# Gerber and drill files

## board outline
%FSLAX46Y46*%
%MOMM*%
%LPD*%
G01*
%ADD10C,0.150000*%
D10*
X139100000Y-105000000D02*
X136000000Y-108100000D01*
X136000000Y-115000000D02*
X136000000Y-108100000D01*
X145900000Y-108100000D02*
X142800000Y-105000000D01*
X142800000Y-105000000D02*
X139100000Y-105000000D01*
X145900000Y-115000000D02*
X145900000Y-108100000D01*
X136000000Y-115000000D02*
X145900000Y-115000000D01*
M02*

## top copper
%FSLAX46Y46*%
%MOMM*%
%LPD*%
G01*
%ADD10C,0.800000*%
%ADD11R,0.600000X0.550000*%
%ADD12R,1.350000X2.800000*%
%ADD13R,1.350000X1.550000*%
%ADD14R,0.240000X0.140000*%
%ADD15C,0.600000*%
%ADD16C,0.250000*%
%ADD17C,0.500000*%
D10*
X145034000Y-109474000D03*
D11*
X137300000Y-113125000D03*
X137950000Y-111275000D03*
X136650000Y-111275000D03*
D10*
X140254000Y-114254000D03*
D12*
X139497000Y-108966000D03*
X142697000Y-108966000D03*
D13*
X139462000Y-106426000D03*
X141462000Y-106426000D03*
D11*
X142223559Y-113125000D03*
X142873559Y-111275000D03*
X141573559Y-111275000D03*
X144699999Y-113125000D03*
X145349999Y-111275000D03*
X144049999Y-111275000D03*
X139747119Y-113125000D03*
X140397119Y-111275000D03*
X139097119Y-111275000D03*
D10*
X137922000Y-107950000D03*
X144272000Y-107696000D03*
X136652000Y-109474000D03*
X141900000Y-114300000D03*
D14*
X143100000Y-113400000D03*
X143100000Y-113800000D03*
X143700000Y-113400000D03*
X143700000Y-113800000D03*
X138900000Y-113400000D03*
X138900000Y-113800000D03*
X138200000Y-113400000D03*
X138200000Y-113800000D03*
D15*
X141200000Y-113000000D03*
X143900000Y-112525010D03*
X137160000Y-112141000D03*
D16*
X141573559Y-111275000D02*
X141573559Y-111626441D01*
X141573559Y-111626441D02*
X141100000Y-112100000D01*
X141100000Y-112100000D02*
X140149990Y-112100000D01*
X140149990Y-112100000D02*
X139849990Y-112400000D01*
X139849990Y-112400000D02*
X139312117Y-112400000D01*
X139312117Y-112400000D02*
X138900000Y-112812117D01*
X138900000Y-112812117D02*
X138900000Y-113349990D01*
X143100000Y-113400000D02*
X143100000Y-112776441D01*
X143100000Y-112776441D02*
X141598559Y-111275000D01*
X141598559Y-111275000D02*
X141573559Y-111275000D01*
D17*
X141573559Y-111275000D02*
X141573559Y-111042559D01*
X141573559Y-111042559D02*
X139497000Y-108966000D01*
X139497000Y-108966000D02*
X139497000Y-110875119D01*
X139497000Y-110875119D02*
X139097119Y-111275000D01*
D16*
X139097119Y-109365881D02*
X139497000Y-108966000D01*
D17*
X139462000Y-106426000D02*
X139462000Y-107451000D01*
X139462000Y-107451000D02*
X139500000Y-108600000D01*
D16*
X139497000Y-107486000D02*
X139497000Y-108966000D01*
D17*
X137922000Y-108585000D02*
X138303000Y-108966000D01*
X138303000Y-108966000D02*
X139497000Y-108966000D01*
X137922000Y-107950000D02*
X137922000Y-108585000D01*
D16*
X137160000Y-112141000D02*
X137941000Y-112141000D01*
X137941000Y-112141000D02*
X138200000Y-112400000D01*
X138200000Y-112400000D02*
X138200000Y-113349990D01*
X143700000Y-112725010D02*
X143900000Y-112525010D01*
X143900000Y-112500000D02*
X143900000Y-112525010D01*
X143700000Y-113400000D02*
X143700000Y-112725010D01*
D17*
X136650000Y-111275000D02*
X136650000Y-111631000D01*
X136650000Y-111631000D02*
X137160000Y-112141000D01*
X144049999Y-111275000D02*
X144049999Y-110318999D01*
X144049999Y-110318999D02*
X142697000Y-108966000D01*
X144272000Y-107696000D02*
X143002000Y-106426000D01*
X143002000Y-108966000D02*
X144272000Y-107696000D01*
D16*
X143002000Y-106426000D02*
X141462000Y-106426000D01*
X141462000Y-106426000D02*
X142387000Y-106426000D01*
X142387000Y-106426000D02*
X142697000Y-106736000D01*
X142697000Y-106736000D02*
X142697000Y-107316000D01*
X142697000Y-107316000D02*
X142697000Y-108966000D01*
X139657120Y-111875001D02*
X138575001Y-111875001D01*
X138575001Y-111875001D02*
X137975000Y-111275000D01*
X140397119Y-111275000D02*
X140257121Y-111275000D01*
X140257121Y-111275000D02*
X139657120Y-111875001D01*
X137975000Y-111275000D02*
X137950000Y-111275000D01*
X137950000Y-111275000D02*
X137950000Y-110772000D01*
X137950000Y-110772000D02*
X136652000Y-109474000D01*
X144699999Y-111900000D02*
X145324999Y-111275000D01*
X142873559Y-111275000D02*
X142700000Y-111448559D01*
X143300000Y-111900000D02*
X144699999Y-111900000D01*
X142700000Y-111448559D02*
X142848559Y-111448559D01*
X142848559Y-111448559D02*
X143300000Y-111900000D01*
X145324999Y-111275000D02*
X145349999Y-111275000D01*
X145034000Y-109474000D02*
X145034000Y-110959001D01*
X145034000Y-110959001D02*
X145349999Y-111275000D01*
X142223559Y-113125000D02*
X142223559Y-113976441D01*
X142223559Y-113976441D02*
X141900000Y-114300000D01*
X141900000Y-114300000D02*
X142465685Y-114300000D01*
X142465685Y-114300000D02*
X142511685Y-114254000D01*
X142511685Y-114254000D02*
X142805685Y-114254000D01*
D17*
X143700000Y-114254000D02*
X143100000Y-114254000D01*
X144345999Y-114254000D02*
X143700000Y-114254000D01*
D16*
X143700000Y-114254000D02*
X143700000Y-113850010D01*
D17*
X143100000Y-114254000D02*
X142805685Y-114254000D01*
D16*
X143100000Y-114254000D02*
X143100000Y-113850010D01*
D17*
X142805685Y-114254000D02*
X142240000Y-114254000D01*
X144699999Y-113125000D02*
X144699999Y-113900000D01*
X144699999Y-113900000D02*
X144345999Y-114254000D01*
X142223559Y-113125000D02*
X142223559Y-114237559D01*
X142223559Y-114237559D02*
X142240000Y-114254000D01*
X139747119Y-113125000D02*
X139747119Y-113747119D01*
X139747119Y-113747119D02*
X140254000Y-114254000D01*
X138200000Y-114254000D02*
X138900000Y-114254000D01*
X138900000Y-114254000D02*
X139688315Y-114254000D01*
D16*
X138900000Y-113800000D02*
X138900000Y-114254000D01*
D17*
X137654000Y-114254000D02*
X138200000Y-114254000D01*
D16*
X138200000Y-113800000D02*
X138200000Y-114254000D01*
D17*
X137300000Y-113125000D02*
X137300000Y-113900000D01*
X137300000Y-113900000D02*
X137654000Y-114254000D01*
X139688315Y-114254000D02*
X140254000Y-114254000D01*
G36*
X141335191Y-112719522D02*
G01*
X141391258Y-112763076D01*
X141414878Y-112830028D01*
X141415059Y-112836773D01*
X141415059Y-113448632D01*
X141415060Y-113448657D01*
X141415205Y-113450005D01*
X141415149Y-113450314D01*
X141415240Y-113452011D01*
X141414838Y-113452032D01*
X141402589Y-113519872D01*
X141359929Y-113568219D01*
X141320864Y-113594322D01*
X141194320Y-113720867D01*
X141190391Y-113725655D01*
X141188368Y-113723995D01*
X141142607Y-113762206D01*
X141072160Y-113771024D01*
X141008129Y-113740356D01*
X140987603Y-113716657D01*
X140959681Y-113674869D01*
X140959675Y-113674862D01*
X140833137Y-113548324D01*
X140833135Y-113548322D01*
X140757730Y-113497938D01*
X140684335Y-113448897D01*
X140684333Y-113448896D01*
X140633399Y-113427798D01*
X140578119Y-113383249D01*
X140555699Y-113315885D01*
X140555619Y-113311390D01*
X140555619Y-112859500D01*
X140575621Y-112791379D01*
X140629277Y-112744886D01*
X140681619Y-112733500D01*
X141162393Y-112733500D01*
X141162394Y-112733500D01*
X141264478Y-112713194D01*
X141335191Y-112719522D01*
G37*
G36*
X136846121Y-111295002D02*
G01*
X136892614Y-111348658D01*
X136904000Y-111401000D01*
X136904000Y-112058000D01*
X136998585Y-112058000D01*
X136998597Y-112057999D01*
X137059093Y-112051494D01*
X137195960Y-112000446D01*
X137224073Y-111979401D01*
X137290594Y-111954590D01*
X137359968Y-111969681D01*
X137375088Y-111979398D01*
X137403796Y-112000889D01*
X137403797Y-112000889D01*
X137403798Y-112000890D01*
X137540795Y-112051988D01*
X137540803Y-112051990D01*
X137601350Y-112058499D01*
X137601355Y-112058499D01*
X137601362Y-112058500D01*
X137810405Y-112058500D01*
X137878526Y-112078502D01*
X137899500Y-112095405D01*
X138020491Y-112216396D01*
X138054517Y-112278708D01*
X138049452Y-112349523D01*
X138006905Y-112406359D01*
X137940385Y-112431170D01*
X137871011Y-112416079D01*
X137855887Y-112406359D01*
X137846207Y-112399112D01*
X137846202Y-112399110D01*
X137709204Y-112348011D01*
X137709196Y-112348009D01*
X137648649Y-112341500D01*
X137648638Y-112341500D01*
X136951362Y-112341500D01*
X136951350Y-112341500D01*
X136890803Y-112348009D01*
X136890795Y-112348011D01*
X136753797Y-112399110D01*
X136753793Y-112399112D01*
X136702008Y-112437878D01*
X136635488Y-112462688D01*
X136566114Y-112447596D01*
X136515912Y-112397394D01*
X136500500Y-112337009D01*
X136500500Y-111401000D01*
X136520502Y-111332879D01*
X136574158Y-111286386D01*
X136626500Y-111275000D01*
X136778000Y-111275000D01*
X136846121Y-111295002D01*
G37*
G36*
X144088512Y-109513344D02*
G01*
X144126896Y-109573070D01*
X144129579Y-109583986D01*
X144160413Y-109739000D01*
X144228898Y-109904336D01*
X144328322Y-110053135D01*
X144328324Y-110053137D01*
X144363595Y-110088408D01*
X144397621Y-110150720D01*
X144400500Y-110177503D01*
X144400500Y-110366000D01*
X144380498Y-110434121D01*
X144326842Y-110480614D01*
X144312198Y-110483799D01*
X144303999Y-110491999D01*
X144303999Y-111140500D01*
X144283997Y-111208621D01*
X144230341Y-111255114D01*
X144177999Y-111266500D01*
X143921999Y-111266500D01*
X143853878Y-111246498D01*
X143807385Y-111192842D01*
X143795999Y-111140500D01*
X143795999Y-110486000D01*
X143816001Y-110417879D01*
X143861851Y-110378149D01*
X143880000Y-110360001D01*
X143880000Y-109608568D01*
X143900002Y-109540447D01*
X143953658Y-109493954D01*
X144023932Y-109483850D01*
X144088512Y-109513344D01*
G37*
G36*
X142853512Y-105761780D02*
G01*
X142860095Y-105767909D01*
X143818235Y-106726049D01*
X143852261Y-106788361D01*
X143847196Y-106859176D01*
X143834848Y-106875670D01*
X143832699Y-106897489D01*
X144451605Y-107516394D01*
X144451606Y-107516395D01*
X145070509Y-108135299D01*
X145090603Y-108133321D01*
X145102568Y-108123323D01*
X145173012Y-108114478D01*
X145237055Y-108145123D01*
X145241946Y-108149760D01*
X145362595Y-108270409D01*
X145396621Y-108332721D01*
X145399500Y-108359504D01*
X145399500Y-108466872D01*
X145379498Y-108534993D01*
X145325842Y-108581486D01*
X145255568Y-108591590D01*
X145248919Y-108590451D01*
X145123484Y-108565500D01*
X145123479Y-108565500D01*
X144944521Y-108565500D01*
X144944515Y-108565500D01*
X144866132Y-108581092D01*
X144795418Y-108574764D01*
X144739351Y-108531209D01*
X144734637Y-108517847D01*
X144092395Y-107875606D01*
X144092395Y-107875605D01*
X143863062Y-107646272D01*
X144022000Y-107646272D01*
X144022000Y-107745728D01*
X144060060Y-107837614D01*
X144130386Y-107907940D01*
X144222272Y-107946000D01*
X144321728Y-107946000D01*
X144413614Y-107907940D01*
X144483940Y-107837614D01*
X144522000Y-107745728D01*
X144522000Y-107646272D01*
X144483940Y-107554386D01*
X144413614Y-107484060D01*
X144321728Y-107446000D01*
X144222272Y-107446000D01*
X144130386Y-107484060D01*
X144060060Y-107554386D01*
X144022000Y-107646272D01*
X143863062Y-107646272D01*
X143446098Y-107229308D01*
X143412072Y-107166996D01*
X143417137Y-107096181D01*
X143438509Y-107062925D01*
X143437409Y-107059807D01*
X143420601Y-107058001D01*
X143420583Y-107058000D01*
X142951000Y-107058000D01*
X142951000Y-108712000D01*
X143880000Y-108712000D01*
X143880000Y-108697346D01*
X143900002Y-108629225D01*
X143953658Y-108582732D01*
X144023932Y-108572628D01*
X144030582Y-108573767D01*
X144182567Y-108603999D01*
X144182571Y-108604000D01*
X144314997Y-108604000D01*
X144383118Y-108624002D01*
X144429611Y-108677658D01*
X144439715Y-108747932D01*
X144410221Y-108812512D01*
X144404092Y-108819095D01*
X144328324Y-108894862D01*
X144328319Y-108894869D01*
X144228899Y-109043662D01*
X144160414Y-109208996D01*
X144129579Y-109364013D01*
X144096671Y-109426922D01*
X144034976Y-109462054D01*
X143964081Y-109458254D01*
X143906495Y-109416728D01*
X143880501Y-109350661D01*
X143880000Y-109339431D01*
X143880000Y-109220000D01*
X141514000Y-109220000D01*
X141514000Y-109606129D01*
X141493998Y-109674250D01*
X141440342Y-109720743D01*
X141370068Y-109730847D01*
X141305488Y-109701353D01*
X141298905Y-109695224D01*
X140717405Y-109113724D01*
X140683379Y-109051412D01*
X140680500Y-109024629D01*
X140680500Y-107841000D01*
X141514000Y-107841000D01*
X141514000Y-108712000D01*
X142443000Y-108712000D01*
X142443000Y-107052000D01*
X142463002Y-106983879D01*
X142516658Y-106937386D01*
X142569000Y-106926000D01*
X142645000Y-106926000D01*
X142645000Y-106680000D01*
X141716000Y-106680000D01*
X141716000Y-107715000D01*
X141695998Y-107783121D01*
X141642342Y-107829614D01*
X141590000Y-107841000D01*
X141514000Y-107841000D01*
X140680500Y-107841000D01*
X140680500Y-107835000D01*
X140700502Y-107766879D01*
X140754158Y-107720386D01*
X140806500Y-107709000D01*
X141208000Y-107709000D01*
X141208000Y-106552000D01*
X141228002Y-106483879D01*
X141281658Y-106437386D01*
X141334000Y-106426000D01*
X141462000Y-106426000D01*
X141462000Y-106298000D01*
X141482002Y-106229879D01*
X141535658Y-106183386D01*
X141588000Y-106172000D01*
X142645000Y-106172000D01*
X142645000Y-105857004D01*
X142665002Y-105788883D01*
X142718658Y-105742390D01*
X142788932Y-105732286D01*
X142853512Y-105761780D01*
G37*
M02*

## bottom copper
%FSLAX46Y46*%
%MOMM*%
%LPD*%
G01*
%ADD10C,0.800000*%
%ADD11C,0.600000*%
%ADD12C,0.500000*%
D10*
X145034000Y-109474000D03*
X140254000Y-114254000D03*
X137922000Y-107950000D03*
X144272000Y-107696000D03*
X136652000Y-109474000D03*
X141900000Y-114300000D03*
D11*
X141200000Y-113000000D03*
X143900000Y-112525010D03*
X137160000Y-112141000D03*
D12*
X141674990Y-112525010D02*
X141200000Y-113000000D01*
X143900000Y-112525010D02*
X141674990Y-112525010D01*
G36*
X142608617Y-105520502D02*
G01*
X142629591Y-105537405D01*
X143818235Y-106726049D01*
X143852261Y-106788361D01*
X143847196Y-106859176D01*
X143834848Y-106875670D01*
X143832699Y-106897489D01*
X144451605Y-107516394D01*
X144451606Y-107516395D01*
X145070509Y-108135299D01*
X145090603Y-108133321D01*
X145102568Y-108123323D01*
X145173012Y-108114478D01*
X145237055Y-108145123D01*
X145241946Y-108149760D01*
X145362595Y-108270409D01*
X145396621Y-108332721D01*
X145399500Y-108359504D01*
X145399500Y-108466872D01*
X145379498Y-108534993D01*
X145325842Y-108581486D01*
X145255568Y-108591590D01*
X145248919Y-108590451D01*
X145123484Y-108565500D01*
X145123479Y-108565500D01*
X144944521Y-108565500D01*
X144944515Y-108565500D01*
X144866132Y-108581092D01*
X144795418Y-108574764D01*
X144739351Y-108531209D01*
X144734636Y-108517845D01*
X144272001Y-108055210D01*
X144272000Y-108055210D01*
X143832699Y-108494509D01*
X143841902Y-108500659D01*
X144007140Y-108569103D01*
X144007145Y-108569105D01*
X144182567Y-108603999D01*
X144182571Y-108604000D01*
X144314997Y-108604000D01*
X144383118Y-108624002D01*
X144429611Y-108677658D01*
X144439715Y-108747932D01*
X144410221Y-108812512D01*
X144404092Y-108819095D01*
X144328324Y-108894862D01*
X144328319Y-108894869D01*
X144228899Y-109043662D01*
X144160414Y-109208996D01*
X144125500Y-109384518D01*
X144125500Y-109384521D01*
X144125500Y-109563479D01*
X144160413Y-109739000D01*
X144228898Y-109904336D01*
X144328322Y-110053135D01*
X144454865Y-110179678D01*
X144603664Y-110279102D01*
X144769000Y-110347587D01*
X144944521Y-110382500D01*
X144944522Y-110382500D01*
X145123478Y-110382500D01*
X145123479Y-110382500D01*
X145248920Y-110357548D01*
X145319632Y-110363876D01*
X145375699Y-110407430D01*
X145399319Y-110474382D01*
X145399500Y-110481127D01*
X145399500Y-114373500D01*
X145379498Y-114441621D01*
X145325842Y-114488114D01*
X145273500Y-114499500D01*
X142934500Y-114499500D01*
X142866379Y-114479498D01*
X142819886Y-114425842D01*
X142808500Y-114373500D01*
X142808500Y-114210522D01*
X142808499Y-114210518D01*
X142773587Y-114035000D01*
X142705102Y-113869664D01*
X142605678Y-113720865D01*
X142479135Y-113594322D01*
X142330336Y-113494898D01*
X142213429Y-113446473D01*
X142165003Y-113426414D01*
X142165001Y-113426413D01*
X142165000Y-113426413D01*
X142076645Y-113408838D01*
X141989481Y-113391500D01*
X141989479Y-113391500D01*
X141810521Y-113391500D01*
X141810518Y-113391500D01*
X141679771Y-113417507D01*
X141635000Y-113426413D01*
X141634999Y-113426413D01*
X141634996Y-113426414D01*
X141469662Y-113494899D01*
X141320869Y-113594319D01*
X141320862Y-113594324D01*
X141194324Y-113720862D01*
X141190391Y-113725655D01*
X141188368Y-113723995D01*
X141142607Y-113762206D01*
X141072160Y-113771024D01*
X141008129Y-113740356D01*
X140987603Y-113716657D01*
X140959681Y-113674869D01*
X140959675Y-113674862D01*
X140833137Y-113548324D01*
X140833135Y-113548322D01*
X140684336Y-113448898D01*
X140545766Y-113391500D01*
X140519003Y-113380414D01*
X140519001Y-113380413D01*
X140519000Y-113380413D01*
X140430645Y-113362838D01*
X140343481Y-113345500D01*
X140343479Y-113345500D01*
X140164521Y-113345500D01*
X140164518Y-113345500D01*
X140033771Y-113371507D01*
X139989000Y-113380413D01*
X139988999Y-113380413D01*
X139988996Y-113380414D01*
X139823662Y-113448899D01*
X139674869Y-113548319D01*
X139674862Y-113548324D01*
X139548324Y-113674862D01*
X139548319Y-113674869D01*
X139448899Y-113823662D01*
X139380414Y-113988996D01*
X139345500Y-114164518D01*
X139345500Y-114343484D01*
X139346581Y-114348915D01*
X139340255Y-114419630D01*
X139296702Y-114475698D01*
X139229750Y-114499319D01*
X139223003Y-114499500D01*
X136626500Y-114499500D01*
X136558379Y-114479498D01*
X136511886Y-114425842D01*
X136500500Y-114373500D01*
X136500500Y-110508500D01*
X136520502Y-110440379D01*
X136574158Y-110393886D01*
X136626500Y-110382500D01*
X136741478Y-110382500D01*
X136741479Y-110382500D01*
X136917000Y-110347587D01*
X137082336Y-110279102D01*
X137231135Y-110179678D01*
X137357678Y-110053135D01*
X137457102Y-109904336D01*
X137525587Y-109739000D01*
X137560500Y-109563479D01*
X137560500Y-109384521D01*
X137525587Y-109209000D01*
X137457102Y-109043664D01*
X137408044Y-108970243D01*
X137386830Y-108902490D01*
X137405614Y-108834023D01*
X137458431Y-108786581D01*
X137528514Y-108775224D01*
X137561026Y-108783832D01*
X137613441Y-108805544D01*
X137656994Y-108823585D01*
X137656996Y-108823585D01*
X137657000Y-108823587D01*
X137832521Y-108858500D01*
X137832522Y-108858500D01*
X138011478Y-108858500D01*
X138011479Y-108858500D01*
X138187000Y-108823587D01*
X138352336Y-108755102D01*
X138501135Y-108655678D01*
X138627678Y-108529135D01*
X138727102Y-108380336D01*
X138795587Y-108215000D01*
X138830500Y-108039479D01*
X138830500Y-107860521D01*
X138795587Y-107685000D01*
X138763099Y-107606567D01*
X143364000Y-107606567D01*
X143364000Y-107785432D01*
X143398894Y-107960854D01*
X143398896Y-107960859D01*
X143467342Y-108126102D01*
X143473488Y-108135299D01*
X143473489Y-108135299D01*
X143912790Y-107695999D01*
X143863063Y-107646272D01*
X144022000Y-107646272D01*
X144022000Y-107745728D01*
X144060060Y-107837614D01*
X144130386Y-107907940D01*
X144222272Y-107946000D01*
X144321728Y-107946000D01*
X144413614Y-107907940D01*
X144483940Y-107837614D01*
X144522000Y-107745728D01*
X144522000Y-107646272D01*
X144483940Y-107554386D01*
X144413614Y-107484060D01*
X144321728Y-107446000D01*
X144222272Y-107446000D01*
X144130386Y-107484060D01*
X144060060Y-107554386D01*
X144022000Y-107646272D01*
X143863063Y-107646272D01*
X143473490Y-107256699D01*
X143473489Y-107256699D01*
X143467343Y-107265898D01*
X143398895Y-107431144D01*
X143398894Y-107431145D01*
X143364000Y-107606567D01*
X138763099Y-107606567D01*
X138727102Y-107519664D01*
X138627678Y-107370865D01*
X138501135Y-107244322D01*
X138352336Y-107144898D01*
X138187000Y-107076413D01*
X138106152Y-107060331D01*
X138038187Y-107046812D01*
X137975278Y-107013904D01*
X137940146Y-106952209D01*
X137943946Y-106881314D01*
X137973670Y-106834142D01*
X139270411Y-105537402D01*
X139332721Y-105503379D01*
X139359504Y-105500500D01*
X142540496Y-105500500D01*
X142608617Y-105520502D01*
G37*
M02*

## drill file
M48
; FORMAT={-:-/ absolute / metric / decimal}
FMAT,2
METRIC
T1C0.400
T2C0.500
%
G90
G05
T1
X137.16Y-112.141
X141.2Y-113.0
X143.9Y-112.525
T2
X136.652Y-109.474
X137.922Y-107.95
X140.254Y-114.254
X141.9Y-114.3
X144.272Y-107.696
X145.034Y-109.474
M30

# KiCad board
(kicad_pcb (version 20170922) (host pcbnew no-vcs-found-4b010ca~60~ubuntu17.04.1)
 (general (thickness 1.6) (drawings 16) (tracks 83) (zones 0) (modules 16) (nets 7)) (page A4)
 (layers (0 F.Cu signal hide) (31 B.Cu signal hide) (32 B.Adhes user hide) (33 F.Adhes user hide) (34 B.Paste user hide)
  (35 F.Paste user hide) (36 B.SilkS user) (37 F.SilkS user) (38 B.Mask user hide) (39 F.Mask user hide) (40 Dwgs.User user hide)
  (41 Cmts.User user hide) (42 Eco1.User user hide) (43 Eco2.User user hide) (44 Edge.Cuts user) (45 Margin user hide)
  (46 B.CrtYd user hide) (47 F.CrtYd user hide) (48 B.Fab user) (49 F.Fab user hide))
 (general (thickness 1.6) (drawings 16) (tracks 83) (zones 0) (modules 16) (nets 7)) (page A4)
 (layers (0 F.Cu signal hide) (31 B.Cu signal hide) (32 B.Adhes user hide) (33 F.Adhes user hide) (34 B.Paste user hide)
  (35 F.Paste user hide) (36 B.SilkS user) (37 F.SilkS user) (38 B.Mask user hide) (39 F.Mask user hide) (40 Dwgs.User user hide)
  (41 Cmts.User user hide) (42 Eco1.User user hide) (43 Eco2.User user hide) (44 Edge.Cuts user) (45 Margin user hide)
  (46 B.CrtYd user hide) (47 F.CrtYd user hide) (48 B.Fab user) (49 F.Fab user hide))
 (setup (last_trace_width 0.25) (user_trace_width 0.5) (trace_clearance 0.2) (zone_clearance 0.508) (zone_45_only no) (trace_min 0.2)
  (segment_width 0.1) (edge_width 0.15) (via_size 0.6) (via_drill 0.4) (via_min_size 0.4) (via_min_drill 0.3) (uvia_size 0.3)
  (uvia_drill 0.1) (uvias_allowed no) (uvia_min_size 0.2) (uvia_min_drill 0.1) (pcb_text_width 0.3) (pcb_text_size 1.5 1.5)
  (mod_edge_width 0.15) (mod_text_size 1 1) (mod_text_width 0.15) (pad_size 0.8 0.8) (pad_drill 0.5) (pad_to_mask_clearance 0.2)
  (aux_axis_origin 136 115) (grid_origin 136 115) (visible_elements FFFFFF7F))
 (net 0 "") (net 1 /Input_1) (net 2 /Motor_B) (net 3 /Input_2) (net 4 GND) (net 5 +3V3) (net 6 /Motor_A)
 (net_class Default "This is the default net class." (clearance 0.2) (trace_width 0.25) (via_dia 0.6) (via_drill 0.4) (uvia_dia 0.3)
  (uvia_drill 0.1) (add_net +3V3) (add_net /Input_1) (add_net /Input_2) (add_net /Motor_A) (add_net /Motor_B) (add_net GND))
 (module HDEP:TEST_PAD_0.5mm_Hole (layer F.Cu) (at 145.034 109.474)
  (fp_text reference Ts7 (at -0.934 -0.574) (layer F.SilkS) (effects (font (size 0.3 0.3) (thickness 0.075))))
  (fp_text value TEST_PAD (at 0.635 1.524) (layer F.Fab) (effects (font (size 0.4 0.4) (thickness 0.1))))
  (pad 1 thru_hole circle (at 0 0) (size 0.8 0.8) (drill 0.5) (layers *.Cu *.Mask F.SilkS) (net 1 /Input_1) (solder_mask_margin 0.1)))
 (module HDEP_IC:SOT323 (layer F.Cu) (at 137.3 112.2 90)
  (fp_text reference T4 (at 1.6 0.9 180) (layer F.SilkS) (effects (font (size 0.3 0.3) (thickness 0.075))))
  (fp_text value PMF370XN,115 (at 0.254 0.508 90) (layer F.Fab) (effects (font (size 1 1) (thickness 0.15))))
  (pad 3 smd rect (at -0.925 0 90) (size 0.55 0.6) (layers F.Cu F.Paste F.Mask) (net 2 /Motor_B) (solder_paste_margin -0.1))
  (pad 1 smd rect (at 0.925 0.65 90) (size 0.55 0.6) (layers F.Cu F.Paste F.Mask) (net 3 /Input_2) (solder_paste_margin -0.1))
  (pad 2 smd rect (at 0.925 -0.65 90) (size 0.55 0.6) (layers F.Cu F.Paste F.Mask) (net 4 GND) (solder_paste_margin -0.1)))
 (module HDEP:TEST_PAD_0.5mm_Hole (layer F.Cu) (at 140.254 114.254)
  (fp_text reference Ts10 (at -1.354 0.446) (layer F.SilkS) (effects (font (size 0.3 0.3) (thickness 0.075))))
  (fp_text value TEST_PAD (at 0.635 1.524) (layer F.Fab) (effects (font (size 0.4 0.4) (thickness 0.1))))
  (pad 1 thru_hole circle (at 0 0) (size 0.8 0.8) (drill 0.5) (layers *.Cu *.Mask F.SilkS) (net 2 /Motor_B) (solder_mask_margin 0.1)))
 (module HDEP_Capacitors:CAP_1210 (layer F.Cu) (at 141.097 108.966)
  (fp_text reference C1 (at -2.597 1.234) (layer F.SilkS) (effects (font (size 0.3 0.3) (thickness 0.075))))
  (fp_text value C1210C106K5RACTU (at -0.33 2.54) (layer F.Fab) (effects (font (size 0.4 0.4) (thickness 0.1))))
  (pad 1 smd rect (at -1.6 0) (size 1.35 2.8) (layers F.Cu F.Paste F.Mask) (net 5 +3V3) (solder_mask_margin 0.102))
  (pad 2 smd rect (at 1.6 0) (size 1.35 2.8) (layers F.Cu F.Paste F.Mask) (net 4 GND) (solder_mask_margin 0.102)))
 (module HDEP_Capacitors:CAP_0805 (layer F.Cu) (at 140.462 106.426)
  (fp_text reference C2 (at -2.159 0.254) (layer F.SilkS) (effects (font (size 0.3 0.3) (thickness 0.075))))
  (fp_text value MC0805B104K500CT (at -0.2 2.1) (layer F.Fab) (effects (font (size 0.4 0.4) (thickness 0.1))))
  (pad 1 smd rect (at -1 0) (size 1.35 1.55) (layers F.Cu F.Paste F.Mask) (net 5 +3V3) (solder_mask_margin 0.102))
  (pad 2 smd rect (at 1 0) (size 1.35 1.55) (layers F.Cu F.Paste F.Mask) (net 4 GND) (solder_mask_margin 0.102)))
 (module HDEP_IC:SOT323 (layer F.Cu) (at 142.223559 112.2 90)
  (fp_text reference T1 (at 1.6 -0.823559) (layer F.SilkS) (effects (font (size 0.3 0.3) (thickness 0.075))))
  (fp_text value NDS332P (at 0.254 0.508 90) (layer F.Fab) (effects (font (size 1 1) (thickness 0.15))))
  (pad 3 smd rect (at -0.925 0 90) (size 0.55 0.6) (layers F.Cu F.Paste F.Mask) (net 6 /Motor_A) (solder_paste_margin -0.1))
  (pad 1 smd rect (at 0.925 0.65 90) (size 0.55 0.6) (layers F.Cu F.Paste F.Mask) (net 1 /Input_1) (solder_paste_margin -0.1))
  (pad 2 smd rect (at 0.925 -0.65 90) (size 0.55 0.6) (layers F.Cu F.Paste F.Mask) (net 5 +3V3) (solder_paste_margin -0.1)))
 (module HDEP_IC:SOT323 (layer F.Cu) (at 144.699999 112.2 90)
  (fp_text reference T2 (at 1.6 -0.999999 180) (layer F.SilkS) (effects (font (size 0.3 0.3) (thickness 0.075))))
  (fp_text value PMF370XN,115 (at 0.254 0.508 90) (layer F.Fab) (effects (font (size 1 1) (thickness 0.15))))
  (pad 3 smd rect (at -0.925 0 90) (size 0.55 0.6) (layers F.Cu F.Paste F.Mask) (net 6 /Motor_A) (solder_paste_margin -0.1))
  (pad 1 smd rect (at 0.925 0.65 90) (size 0.55 0.6) (layers F.Cu F.Paste F.Mask) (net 1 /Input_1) (solder_paste_margin -0.1))
  (pad 2 smd rect (at 0.925 -0.65 90) (size 0.55 0.6) (layers F.Cu F.Paste F.Mask) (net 4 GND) (solder_paste_margin -0.1)))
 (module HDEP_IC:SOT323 (layer F.Cu) (at 139.747119 112.2 90)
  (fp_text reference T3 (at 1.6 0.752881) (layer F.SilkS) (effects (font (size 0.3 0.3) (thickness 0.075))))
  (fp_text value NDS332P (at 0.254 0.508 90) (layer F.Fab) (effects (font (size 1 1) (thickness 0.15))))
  (pad 3 smd rect (at -0.925 0 90) (size 0.55 0.6) (layers F.Cu F.Paste F.Mask) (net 2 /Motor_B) (solder_paste_margin -0.1))
  (pad 1 smd rect (at 0.925 0.65 90) (size 0.55 0.6) (layers F.Cu F.Paste F.Mask) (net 3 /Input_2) (solder_paste_margin -0.1))
  (pad 2 smd rect (at 0.925 -0.65 90) (size 0.55 0.6) (layers F.Cu F.Paste F.Mask) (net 5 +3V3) (solder_paste_margin -0.1)))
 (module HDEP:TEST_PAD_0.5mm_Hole (layer F.Cu) (at 137.922 107.95)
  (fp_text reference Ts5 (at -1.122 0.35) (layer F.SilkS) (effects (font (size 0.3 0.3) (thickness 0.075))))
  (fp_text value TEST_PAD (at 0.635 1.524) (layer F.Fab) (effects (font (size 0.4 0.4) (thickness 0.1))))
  (pad 1 thru_hole circle (at 0 0) (size 0.8 0.8) (drill 0.5) (layers *.Cu *.Mask F.SilkS) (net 5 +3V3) (solder_mask_margin 0.1)))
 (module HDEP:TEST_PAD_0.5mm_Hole (layer F.Cu) (at 144.272 107.696)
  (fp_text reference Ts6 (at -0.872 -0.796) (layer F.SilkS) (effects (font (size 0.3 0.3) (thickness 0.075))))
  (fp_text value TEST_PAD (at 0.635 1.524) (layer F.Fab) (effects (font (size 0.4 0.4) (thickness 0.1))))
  (pad 1 thru_hole circle (at 0 0) (size 0.8 0.8) (drill 0.5) (layers *.Cu *.Mask F.SilkS) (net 4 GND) (solder_mask_margin 0.1)))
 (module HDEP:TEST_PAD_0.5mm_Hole (layer F.Cu) (at 136.652 109.474)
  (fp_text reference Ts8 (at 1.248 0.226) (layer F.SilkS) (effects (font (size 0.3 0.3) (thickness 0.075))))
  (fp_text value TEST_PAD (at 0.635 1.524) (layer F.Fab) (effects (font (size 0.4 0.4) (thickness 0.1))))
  (pad 1 thru_hole circle (at 0 0) (size 0.8 0.8) (drill 0.5) (layers *.Cu *.Mask F.SilkS) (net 3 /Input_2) (solder_mask_margin 0.1)))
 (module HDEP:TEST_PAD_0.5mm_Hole (layer F.Cu) (at 141.9 114.3)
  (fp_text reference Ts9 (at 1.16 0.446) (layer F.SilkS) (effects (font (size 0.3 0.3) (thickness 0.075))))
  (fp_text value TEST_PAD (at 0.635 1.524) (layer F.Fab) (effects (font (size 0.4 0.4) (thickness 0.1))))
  (pad 1 thru_hole circle (at 0 0) (size 0.8 0.8) (drill 0.5) (layers *.Cu *.Mask F.SilkS) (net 6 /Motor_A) (solder_mask_margin 0.1)))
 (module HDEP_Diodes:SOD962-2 (layer F.Cu) (at 143.1 113.6 270)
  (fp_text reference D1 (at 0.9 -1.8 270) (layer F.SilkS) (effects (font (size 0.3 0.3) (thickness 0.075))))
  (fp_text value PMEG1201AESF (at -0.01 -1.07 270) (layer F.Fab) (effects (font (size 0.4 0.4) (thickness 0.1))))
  (pad 1 smd rect (at -0.2 0 270) (size 0.14 0.24) (layers F.Cu F.Paste F.Mask) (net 5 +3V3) (solder_mask_margin 0.05))
  (pad 2 smd rect (at 0.2 0 270) (size 0.14 0.24) (layers F.Cu F.Paste F.Mask) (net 6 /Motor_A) (solder_mask_margin 0.05)))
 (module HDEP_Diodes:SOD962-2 (layer F.Cu) (at 143.7 113.6 90)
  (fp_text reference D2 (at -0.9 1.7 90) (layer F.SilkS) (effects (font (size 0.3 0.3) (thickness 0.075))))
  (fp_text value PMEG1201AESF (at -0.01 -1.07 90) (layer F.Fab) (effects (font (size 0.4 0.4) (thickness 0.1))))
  (pad 2 smd rect (at 0.2 0 90) (size 0.14 0.24) (layers F.Cu F.Paste F.Mask) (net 4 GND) (solder_mask_margin 0.05))
  (pad 1 smd rect (at -0.2 0 90) (size 0.14 0.24) (layers F.Cu F.Paste F.Mask) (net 6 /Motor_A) (solder_mask_margin 0.05)))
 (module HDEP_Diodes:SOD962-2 (layer F.Cu) (at 138.9 113.6 270)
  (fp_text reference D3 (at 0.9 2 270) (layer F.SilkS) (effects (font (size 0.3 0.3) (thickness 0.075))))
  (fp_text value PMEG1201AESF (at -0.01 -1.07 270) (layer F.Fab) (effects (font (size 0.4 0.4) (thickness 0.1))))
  (pad 1 smd rect (at -0.2 0 270) (size 0.14 0.24) (layers F.Cu F.Paste F.Mask) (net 5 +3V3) (solder_mask_margin 0.05))
  (pad 2 smd rect (at 0.2 0 270) (size 0.14 0.24) (layers F.Cu F.Paste F.Mask) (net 2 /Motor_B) (solder_mask_margin 0.05)))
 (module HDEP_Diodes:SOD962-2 (layer F.Cu) (at 138.2 113.6 90)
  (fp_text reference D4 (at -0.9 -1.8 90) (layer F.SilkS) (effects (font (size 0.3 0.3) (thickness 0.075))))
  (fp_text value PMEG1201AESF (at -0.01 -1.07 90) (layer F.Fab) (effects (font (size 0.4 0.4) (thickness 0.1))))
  (pad 2 smd rect (at 0.2 0 90) (size 0.14 0.24) (layers F.Cu F.Paste F.Mask) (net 4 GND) (solder_mask_margin 0.05))
  (pad 1 smd rect (at -0.2 0 90) (size 0.14 0.24) (layers F.Cu F.Paste F.Mask) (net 2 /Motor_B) (solder_mask_margin 0.05)))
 (gr_line (start 139.1 105) (end 136 108.1) (layer Edge.Cuts) (width 0.15))
 (gr_line (start 136 115) (end 136 108.1) (layer Edge.Cuts) (width 0.15))
 (gr_line (start 145.9 108.1) (end 142.8 105) (layer Edge.Cuts) (width 0.15))
 (gr_line (start 142.8 105) (end 139.1 105) (layer Edge.Cuts) (width 0.15))
 (gr_line (start 145.9 115) (end 145.9 108.1) (layer Edge.Cuts) (width 0.15))
 (gr_line (start 136 115) (end 145.9 115) (layer Edge.Cuts) (width 0.15))
 (segment (start 141.573559 111.275) (end 141.573559 111.626441) (width 0.25) (layer F.Cu) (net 5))
 (segment (start 141.573559 111.626441) (end 141.1 112.1) (width 0.25) (layer F.Cu) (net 5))
 (segment (start 141.1 112.1) (end 140.14999 112.1) (width 0.25) (layer F.Cu) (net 5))
 (segment (start 140.14999 112.1) (end 139.84999 112.4) (width 0.25) (layer F.Cu) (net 5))
 (segment (start 139.84999 112.4) (end 139.312117 112.4) (width 0.25) (layer F.Cu) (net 5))
 (segment (start 139.312117 112.4) (end 138.9 112.812117) (width 0.25) (layer F.Cu) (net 5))
 (segment (start 138.9 112.812117) (end 138.9 113.34999) (width 0.25) (layer F.Cu) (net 5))
 (segment (start 143.1 113.4) (end 143.1 112.776441) (width 0.25) (layer F.Cu) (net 5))
 (segment (start 143.1 112.776441) (end 141.598559 111.275) (width 0.25) (layer F.Cu) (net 5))
 (segment (start 141.598559 111.275) (end 141.573559 111.275) (width 0.25) (layer F.Cu) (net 5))
 (segment (start 141.573559 111.275) (end 141.573559 111.042559) (width 0.5) (layer F.Cu) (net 5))
 (segment (start 141.573559 111.042559) (end 139.497 108.966) (width 0.5) (layer F.Cu) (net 5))
 (segment (start 139.497 108.966) (end 139.497 110.875119) (width 0.5) (layer F.Cu) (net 5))
 (segment (start 139.497 110.875119) (end 139.097119 111.275) (width 0.5) (layer F.Cu) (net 5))
 (segment (start 139.097119 109.365881) (end 139.497 108.966) (width 0.25) (layer F.Cu) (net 5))
 (segment (start 139.462 106.426) (end 139.462 107.451) (width 0.5) (layer F.Cu) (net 5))
 (segment (start 139.462 107.451) (end 139.5 108.6) (width 0.5) (layer F.Cu) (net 5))
 (segment (start 139.497 107.486) (end 139.497 108.966) (width 0.25) (layer F.Cu) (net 5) (status 20))
 (segment (start 137.922 108.585) (end 138.303 108.966) (width 0.5) (layer F.Cu) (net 5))
 (segment (start 138.303 108.966) (end 139.497 108.966) (width 0.5) (layer F.Cu) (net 5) (status 20))
 (segment (start 137.922 107.95) (end 137.922 108.585) (width 0.5) (layer F.Cu) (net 5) (status 10))
 (via (at 141.2 113) (size 0.6) (drill 0.4) (layers F.Cu B.Cu) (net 4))
 (segment (start 141.67499 112.52501) (end 141.2 113) (width 0.5) (layer B.Cu) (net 4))
 (segment (start 143.9 112.52501) (end 141.67499 112.52501) (width 0.5) (layer B.Cu) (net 4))
 (segment (start 137.16 112.141) (end 137.941 112.141) (width 0.25) (layer F.Cu) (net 4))
 (segment (start 137.941 112.141) (end 138.2 112.4) (width 0.25) (layer F.Cu) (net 4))
 (segment (start 138.2 112.4) (end 138.2 113.34999) (width 0.25) (layer F.Cu) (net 4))
 (segment (start 143.7 112.72501) (end 143.9 112.52501) (width 0.25) (layer F.Cu) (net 4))
 (segment (start 143.9 112.5) (end 143.9 112.52501) (width 0.25) (layer F.Cu) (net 4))
 (via (at 143.9 112.52501) (size 0.6) (drill 0.4) (layers F.Cu B.Cu) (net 4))
 (segment (start 143.7 113.4) (end 143.7 112.72501) (width 0.25) (layer F.Cu) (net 4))
 (segment (start 136.65 111.275) (end 136.65 111.631) (width 0.5) (layer F.Cu) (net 4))
 (segment (start 136.65 111.631) (end 137.16 112.141) (width 0.5) (layer F.Cu) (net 4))
 (segment (start 144.049999 111.275) (end 144.049999 110.318999) (width 0.5) (layer F.Cu) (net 4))
 (segment (start 144.049999 110.318999) (end 142.697 108.966) (width 0.5) (layer F.Cu) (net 4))
 (segment (start 144.272 107.696) (end 143.002 106.426) (width 0.5) (layer F.Cu) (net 4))
 (segment (start 143.002 108.966) (end 144.272 107.696) (width 0.5) (layer F.Cu) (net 4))
 (via (at 137.16 112.141) (size 0.6) (drill 0.4) (layers F.Cu B.Cu) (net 4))
 (segment (start 143.002 106.426) (end 141.462 106.426) (width 0.25) (layer F.Cu) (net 4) (status 20))
 (segment (start 141.462 106.426) (end 142.387 106.426) (width 0.25) (layer F.Cu) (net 4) (status 10))
 (segment (start 142.387 106.426) (end 142.697 106.736) (width 0.25) (layer F.Cu) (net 4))
 (segment (start 142.697 106.736) (end 142.697 107.316) (width 0.25) (layer F.Cu) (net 4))
 (segment (start 142.697 107.316) (end 142.697 108.966) (width 0.25) (layer F.Cu) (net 4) (status 20))
 (segment (start 139.65712 111.875001) (end 138.575001 111.875001) (width 0.25) (layer F.Cu) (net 3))
 (segment (start 138.575001 111.875001) (end 137.975 111.275) (width 0.25) (layer F.Cu) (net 3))
 (segment (start 140.397119 111.275) (end 140.257121 111.275) (width 0.25) (layer F.Cu) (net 3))
 (segment (start 140.257121 111.275) (end 139.65712 111.875001) (width 0.25) (layer F.Cu) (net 3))
 (segment (start 137.975 111.275) (end 137.95 111.275) (width 0.25) (layer F.Cu) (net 3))
 (segment (start 137.95 111.275) (end 137.95 110.772) (width 0.25) (layer F.Cu) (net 3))
 (segment (start 137.95 110.772) (end 136.652 109.474) (width 0.25) (layer F.Cu) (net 3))
 (segment (start 144.699999 111.9) (end 145.324999 111.275) (width 0.25) (layer F.Cu) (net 1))
 (segment (start 142.873559 111.275) (end 142.7 111.448559) (width 0.25) (layer F.Cu) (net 1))
 (segment (start 143.3 111.9) (end 144.699999 111.9) (width 0.25) (layer F.Cu) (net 1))
 (segment (start 142.7 111.448559) (end 142.848559 111.448559) (width 0.25) (layer F.Cu) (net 1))
 (segment (start 142.848559 111.448559) (end 143.3 111.9) (width 0.25) (layer F.Cu) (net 1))
 (segment (start 145.324999 111.275) (end 145.349999 111.275) (width 0.25) (layer F.Cu) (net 1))
 (segment (start 145.034 109.474) (end 145.034 110.959001) (width 0.25) (layer F.Cu) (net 1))
 (segment (start 145.034 110.959001) (end 145.349999 111.275) (width 0.25) (layer F.Cu) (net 1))
 (segment (start 142.223559 113.125) (end 142.223559 113.976441) (width 0.25) (layer F.Cu) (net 6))
 (segment (start 142.223559 113.976441) (end 141.9 114.3) (width 0.25) (layer F.Cu) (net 6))
 (segment (start 141.9 114.3) (end 142.465685 114.3) (width 0.25) (layer F.Cu) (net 6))
 (segment (start 142.465685 114.3) (end 142.511685 114.254) (width 0.25) (layer F.Cu) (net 6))
 (segment (start 142.511685 114.254) (end 142.805685 114.254) (width 0.25) (layer F.Cu) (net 6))
 (segment (start 143.7 114.254) (end 143.1 114.254) (width 0.5) (layer F.Cu) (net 6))
 (segment (start 144.345999 114.254) (end 143.7 114.254) (width 0.5) (layer F.Cu) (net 6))
 (segment (start 143.7 114.254) (end 143.7 113.85001) (width 0.25) (layer F.Cu) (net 6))
 (segment (start 143.1 114.254) (end 142.805685 114.254) (width 0.5) (layer F.Cu) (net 6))
 (segment (start 143.1 114.254) (end 143.1 113.85001) (width 0.25) (layer F.Cu) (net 6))
 (segment (start 142.805685 114.254) (end 142.24 114.254) (width 0.5) (layer F.Cu) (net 6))
 (segment (start 144.699999 113.125) (end 144.699999 113.9) (width 0.5) (layer F.Cu) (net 6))
 (segment (start 144.699999 113.9) (end 144.345999 114.254) (width 0.5) (layer F.Cu) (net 6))
 (segment (start 142.223559 113.125) (end 142.223559 114.237559) (width 0.5) (layer F.Cu) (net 6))
 (segment (start 142.223559 114.237559) (end 142.24 114.254) (width 0.5) (layer F.Cu) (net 6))
 (segment (start 139.747119 113.125) (end 139.747119 113.747119) (width 0.5) (layer F.Cu) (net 2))
 (segment (start 139.747119 113.747119) (end 140.254 114.254) (width 0.5) (layer F.Cu) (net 2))
 (segment (start 138.2 114.254) (end 138.9 114.254) (width 0.5) (layer F.Cu) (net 2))
 (segment (start 138.9 114.254) (end 139.688315 114.254) (width 0.5) (layer F.Cu) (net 2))
 (segment (start 138.9 113.8) (end 138.9 114.254) (width 0.25) (layer F.Cu) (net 2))
 (segment (start 137.654 114.254) (end 138.2 114.254) (width 0.5) (layer F.Cu) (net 2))
 (segment (start 138.2 113.8) (end 138.2 114.254) (width 0.25) (layer F.Cu) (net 2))
 (segment (start 137.3 113.125) (end 137.3 113.9) (width 0.5) (layer F.Cu) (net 2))
 (segment (start 137.3 113.9) (end 137.654 114.254) (width 0.5) (layer F.Cu) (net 2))
 (segment (start 139.688315 114.254) (end 140.254 114.254) (width 0.5) (layer F.Cu) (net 2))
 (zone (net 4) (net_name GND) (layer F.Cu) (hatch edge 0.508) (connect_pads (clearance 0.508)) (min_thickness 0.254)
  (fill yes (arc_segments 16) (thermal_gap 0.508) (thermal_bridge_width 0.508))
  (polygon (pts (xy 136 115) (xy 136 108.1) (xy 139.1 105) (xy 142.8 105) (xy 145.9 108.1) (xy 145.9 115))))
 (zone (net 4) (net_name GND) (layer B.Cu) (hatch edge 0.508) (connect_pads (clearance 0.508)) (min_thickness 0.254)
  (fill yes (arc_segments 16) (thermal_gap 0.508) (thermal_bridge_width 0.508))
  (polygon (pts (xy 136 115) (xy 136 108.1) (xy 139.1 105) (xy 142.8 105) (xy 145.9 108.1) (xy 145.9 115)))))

